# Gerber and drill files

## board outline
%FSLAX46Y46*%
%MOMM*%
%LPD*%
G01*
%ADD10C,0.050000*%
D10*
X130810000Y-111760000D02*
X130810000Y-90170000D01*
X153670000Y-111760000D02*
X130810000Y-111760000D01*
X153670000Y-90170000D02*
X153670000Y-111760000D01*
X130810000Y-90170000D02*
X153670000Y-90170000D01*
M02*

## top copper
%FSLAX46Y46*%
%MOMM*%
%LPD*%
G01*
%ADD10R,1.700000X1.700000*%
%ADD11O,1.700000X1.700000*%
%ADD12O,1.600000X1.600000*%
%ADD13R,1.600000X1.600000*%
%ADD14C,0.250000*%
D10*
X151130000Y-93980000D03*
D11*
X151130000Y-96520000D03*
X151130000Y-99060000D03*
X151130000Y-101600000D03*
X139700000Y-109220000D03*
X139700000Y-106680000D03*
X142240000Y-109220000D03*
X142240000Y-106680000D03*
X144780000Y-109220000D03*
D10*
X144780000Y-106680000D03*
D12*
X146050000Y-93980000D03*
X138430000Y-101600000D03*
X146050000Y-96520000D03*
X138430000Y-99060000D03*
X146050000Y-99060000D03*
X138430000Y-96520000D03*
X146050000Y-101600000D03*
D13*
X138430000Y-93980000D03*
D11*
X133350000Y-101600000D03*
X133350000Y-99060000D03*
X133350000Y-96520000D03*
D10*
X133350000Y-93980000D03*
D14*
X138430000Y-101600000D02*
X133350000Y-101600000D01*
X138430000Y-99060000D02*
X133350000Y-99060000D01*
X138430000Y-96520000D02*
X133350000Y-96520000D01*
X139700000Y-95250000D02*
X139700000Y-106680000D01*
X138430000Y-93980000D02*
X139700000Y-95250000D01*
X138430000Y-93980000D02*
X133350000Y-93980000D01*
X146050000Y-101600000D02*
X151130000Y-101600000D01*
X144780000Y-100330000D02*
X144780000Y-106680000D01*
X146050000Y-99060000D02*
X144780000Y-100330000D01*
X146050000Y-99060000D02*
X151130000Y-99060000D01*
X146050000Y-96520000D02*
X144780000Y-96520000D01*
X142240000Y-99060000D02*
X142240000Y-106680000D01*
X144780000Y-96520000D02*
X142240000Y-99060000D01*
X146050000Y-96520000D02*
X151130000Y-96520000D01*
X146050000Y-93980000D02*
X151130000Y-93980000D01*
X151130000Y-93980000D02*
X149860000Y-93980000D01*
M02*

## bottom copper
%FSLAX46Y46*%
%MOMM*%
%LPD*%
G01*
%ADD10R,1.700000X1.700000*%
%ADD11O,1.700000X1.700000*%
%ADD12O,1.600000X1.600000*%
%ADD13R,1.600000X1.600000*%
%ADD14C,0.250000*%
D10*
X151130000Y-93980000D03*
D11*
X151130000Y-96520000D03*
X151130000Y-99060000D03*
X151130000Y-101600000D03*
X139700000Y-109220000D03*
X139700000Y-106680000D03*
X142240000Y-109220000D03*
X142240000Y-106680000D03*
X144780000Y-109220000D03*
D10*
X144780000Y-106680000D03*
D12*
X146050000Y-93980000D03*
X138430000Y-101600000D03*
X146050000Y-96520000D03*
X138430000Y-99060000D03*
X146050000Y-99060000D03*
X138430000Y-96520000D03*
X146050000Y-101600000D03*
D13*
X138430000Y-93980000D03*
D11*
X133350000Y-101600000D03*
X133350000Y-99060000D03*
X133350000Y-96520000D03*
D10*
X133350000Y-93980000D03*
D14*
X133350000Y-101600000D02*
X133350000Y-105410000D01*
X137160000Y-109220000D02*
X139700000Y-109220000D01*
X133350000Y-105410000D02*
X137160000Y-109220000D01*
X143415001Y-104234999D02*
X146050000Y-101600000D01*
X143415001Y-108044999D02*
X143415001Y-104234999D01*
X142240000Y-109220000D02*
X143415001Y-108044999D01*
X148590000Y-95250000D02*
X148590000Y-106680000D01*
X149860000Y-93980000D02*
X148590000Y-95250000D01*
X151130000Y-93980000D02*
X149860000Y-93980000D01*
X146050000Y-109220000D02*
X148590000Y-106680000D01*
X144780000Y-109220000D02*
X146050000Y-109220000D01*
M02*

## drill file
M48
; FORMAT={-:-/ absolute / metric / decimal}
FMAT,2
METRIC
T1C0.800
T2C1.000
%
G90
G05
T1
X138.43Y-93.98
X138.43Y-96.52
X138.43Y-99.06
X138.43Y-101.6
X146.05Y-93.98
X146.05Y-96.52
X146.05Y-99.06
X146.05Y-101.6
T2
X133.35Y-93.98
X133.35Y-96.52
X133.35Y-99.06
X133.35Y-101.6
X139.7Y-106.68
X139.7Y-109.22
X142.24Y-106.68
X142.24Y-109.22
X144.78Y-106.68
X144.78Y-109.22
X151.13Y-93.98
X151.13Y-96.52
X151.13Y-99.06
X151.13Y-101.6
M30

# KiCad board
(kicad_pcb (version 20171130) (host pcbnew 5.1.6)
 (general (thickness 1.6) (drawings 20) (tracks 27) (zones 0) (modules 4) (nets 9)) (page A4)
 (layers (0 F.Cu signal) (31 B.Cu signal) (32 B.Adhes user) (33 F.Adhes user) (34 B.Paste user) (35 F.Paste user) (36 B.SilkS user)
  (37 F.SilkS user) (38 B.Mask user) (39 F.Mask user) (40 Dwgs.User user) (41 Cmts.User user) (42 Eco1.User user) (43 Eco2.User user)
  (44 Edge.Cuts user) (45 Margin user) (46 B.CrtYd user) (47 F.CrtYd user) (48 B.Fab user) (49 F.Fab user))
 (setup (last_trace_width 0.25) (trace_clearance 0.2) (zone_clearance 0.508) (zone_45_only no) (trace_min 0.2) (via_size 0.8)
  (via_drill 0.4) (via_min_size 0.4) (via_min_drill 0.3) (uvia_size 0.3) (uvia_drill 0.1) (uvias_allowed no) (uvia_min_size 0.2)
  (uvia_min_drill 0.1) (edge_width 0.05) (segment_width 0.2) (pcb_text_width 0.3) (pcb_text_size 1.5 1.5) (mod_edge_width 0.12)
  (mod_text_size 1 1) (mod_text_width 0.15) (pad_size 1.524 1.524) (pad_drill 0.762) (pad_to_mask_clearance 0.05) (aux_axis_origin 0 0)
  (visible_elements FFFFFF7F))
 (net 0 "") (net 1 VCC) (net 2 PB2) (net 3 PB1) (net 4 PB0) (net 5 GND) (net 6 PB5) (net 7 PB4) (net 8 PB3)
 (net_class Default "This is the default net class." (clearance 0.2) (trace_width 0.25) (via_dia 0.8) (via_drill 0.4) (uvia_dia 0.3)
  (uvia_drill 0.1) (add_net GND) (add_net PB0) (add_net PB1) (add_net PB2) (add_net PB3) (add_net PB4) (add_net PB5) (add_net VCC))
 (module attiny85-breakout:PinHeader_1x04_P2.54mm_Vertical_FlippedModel (layer F.Cu) (at 151.13 93.98)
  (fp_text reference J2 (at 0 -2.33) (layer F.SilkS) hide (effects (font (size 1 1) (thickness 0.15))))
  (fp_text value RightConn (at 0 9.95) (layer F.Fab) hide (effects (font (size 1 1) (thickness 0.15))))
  (pad 1 thru_hole rect (at 0 0) (size 1.7 1.7) (drill 1) (layers *.Cu *.Mask) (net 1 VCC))
  (pad 2 thru_hole oval (at 0 2.54) (size 1.7 1.7) (drill 1) (layers *.Cu *.Mask) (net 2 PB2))
  (pad 3 thru_hole oval (at 0 5.08) (size 1.7 1.7) (drill 1) (layers *.Cu *.Mask) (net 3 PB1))
  (pad 4 thru_hole oval (at 0 7.62) (size 1.7 1.7) (drill 1) (layers *.Cu *.Mask) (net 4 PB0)))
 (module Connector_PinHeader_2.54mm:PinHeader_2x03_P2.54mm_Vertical (layer F.Cu) (at 144.78 106.68 270)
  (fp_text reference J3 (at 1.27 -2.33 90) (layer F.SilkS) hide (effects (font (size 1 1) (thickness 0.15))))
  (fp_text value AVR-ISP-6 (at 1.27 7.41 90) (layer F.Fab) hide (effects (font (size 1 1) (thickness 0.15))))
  (pad 6 thru_hole oval (at 2.54 5.08 270) (size 1.7 1.7) (drill 1) (layers *.Cu *.Mask) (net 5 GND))
  (pad 5 thru_hole oval (at 0 5.08 270) (size 1.7 1.7) (drill 1) (layers *.Cu *.Mask) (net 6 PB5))
  (pad 4 thru_hole oval (at 2.54 2.54 270) (size 1.7 1.7) (drill 1) (layers *.Cu *.Mask) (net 4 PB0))
  (pad 3 thru_hole oval (at 0 2.54 270) (size 1.7 1.7) (drill 1) (layers *.Cu *.Mask) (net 2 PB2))
  (pad 2 thru_hole oval (at 2.54 0 270) (size 1.7 1.7) (drill 1) (layers *.Cu *.Mask) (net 1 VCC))
  (pad 1 thru_hole rect (at 0 0 270) (size 1.7 1.7) (drill 1) (layers *.Cu *.Mask) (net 3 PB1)))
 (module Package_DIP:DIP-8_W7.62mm (layer F.Cu) (at 138.43 93.98)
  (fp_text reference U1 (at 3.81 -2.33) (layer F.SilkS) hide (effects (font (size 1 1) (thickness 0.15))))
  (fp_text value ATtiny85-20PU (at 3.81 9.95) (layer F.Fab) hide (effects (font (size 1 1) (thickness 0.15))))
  (pad 8 thru_hole oval (at 7.62 0) (size 1.6 1.6) (drill 0.8) (layers *.Cu *.Mask) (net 1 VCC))
  (pad 4 thru_hole oval (at 0 7.62) (size 1.6 1.6) (drill 0.8) (layers *.Cu *.Mask) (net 5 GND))
  (pad 7 thru_hole oval (at 7.62 2.54) (size 1.6 1.6) (drill 0.8) (layers *.Cu *.Mask) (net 2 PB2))
  (pad 3 thru_hole oval (at 0 5.08) (size 1.6 1.6) (drill 0.8) (layers *.Cu *.Mask) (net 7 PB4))
  (pad 6 thru_hole oval (at 7.62 5.08) (size 1.6 1.6) (drill 0.8) (layers *.Cu *.Mask) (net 3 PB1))
  (pad 2 thru_hole oval (at 0 2.54) (size 1.6 1.6) (drill 0.8) (layers *.Cu *.Mask) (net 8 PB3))
  (pad 5 thru_hole oval (at 7.62 7.62) (size 1.6 1.6) (drill 0.8) (layers *.Cu *.Mask) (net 4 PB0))
  (pad 1 thru_hole rect (at 0 0) (size 1.6 1.6) (drill 0.8) (layers *.Cu *.Mask) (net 6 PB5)))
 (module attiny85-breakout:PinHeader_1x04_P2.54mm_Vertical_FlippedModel (layer F.Cu) (at 133.35 93.98)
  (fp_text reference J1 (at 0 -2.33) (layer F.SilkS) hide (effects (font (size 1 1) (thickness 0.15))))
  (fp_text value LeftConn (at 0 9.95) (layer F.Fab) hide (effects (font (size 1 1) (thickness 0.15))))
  (pad 4 thru_hole oval (at 0 7.62) (size 1.7 1.7) (drill 1) (layers *.Cu *.Mask) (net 5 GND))
  (pad 3 thru_hole oval (at 0 5.08) (size 1.7 1.7) (drill 1) (layers *.Cu *.Mask) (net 7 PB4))
  (pad 2 thru_hole oval (at 0 2.54) (size 1.7 1.7) (drill 1) (layers *.Cu *.Mask) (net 8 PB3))
  (pad 1 thru_hole rect (at 0 0) (size 1.7 1.7) (drill 1) (layers *.Cu *.Mask) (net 6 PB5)))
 (gr_line (start 130.81 111.76) (end 130.81 90.17) (layer Edge.Cuts) (width 0.05))
 (gr_line (start 153.67 111.76) (end 130.81 111.76) (layer Edge.Cuts) (width 0.05))
 (gr_line (start 153.67 90.17) (end 153.67 111.76) (layer Edge.Cuts) (width 0.05))
 (gr_line (start 130.81 90.17) (end 153.67 90.17) (layer Edge.Cuts) (width 0.05))
 (segment (start 138.43 101.6) (end 133.35 101.6) (width 0.25) (layer F.Cu) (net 5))
 (segment (start 133.35 101.6) (end 133.35 105.41) (width 0.25) (layer B.Cu) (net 5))
 (segment (start 137.16 109.22) (end 139.7 109.22) (width 0.25) (layer B.Cu) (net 5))
 (segment (start 133.35 105.41) (end 137.16 109.22) (width 0.25) (layer B.Cu) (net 5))
 (segment (start 138.43 99.06) (end 133.35 99.06) (width 0.25) (layer F.Cu) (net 7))
 (segment (start 138.43 96.52) (end 133.35 96.52) (width 0.25) (layer F.Cu) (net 8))
 (segment (start 139.7 95.25) (end 139.7 106.68) (width 0.25) (layer F.Cu) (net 6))
 (segment (start 138.43 93.98) (end 139.7 95.25) (width 0.25) (layer F.Cu) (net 6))
 (segment (start 138.43 93.98) (end 133.35 93.98) (width 0.25) (layer F.Cu) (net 6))
 (segment (start 146.05 101.6) (end 151.13 101.6) (width 0.25) (layer F.Cu) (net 4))
 (segment (start 143.415001 104.234999) (end 146.05 101.6) (width 0.25) (layer B.Cu) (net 4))
 (segment (start 143.415001 108.044999) (end 143.415001 104.234999) (width 0.25) (layer B.Cu) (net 4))
 (segment (start 142.24 109.22) (end 143.415001 108.044999) (width 0.25) (layer B.Cu) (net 4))
 (segment (start 144.78 100.33) (end 144.78 106.68) (width 0.25) (layer F.Cu) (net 3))
 (segment (start 146.05 99.06) (end 144.78 100.33) (width 0.25) (layer F.Cu) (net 3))
 (segment (start 146.05 99.06) (end 151.13 99.06) (width 0.25) (layer F.Cu) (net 3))
 (segment (start 146.05 96.52) (end 144.78 96.52) (width 0.25) (layer F.Cu) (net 2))
 (segment (start 142.24 99.06) (end 142.24 106.68) (width 0.25) (layer F.Cu) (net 2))
 (segment (start 144.78 96.52) (end 142.24 99.06) (width 0.25) (layer F.Cu) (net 2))
 (segment (start 146.05 96.52) (end 151.13 96.52) (width 0.25) (layer F.Cu) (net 2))
 (segment (start 146.05 93.98) (end 151.13 93.98) (width 0.25) (layer F.Cu) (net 1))
 (segment (start 151.13 93.98) (end 149.86 93.98) (width 0.25) (layer F.Cu) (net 1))
 (segment (start 148.59 95.25) (end 148.59 106.68) (width 0.25) (layer B.Cu) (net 1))
 (segment (start 149.86 93.98) (end 148.59 95.25) (width 0.25) (layer B.Cu) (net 1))
 (segment (start 151.13 93.98) (end 149.86 93.98) (width 0.25) (layer B.Cu) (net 1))
 (segment (start 146.05 109.22) (end 148.59 106.68) (width 0.25) (layer B.Cu) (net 1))
 (segment (start 144.78 109.22) (end 146.05 109.22) (width 0.25) (layer B.Cu) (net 1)))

